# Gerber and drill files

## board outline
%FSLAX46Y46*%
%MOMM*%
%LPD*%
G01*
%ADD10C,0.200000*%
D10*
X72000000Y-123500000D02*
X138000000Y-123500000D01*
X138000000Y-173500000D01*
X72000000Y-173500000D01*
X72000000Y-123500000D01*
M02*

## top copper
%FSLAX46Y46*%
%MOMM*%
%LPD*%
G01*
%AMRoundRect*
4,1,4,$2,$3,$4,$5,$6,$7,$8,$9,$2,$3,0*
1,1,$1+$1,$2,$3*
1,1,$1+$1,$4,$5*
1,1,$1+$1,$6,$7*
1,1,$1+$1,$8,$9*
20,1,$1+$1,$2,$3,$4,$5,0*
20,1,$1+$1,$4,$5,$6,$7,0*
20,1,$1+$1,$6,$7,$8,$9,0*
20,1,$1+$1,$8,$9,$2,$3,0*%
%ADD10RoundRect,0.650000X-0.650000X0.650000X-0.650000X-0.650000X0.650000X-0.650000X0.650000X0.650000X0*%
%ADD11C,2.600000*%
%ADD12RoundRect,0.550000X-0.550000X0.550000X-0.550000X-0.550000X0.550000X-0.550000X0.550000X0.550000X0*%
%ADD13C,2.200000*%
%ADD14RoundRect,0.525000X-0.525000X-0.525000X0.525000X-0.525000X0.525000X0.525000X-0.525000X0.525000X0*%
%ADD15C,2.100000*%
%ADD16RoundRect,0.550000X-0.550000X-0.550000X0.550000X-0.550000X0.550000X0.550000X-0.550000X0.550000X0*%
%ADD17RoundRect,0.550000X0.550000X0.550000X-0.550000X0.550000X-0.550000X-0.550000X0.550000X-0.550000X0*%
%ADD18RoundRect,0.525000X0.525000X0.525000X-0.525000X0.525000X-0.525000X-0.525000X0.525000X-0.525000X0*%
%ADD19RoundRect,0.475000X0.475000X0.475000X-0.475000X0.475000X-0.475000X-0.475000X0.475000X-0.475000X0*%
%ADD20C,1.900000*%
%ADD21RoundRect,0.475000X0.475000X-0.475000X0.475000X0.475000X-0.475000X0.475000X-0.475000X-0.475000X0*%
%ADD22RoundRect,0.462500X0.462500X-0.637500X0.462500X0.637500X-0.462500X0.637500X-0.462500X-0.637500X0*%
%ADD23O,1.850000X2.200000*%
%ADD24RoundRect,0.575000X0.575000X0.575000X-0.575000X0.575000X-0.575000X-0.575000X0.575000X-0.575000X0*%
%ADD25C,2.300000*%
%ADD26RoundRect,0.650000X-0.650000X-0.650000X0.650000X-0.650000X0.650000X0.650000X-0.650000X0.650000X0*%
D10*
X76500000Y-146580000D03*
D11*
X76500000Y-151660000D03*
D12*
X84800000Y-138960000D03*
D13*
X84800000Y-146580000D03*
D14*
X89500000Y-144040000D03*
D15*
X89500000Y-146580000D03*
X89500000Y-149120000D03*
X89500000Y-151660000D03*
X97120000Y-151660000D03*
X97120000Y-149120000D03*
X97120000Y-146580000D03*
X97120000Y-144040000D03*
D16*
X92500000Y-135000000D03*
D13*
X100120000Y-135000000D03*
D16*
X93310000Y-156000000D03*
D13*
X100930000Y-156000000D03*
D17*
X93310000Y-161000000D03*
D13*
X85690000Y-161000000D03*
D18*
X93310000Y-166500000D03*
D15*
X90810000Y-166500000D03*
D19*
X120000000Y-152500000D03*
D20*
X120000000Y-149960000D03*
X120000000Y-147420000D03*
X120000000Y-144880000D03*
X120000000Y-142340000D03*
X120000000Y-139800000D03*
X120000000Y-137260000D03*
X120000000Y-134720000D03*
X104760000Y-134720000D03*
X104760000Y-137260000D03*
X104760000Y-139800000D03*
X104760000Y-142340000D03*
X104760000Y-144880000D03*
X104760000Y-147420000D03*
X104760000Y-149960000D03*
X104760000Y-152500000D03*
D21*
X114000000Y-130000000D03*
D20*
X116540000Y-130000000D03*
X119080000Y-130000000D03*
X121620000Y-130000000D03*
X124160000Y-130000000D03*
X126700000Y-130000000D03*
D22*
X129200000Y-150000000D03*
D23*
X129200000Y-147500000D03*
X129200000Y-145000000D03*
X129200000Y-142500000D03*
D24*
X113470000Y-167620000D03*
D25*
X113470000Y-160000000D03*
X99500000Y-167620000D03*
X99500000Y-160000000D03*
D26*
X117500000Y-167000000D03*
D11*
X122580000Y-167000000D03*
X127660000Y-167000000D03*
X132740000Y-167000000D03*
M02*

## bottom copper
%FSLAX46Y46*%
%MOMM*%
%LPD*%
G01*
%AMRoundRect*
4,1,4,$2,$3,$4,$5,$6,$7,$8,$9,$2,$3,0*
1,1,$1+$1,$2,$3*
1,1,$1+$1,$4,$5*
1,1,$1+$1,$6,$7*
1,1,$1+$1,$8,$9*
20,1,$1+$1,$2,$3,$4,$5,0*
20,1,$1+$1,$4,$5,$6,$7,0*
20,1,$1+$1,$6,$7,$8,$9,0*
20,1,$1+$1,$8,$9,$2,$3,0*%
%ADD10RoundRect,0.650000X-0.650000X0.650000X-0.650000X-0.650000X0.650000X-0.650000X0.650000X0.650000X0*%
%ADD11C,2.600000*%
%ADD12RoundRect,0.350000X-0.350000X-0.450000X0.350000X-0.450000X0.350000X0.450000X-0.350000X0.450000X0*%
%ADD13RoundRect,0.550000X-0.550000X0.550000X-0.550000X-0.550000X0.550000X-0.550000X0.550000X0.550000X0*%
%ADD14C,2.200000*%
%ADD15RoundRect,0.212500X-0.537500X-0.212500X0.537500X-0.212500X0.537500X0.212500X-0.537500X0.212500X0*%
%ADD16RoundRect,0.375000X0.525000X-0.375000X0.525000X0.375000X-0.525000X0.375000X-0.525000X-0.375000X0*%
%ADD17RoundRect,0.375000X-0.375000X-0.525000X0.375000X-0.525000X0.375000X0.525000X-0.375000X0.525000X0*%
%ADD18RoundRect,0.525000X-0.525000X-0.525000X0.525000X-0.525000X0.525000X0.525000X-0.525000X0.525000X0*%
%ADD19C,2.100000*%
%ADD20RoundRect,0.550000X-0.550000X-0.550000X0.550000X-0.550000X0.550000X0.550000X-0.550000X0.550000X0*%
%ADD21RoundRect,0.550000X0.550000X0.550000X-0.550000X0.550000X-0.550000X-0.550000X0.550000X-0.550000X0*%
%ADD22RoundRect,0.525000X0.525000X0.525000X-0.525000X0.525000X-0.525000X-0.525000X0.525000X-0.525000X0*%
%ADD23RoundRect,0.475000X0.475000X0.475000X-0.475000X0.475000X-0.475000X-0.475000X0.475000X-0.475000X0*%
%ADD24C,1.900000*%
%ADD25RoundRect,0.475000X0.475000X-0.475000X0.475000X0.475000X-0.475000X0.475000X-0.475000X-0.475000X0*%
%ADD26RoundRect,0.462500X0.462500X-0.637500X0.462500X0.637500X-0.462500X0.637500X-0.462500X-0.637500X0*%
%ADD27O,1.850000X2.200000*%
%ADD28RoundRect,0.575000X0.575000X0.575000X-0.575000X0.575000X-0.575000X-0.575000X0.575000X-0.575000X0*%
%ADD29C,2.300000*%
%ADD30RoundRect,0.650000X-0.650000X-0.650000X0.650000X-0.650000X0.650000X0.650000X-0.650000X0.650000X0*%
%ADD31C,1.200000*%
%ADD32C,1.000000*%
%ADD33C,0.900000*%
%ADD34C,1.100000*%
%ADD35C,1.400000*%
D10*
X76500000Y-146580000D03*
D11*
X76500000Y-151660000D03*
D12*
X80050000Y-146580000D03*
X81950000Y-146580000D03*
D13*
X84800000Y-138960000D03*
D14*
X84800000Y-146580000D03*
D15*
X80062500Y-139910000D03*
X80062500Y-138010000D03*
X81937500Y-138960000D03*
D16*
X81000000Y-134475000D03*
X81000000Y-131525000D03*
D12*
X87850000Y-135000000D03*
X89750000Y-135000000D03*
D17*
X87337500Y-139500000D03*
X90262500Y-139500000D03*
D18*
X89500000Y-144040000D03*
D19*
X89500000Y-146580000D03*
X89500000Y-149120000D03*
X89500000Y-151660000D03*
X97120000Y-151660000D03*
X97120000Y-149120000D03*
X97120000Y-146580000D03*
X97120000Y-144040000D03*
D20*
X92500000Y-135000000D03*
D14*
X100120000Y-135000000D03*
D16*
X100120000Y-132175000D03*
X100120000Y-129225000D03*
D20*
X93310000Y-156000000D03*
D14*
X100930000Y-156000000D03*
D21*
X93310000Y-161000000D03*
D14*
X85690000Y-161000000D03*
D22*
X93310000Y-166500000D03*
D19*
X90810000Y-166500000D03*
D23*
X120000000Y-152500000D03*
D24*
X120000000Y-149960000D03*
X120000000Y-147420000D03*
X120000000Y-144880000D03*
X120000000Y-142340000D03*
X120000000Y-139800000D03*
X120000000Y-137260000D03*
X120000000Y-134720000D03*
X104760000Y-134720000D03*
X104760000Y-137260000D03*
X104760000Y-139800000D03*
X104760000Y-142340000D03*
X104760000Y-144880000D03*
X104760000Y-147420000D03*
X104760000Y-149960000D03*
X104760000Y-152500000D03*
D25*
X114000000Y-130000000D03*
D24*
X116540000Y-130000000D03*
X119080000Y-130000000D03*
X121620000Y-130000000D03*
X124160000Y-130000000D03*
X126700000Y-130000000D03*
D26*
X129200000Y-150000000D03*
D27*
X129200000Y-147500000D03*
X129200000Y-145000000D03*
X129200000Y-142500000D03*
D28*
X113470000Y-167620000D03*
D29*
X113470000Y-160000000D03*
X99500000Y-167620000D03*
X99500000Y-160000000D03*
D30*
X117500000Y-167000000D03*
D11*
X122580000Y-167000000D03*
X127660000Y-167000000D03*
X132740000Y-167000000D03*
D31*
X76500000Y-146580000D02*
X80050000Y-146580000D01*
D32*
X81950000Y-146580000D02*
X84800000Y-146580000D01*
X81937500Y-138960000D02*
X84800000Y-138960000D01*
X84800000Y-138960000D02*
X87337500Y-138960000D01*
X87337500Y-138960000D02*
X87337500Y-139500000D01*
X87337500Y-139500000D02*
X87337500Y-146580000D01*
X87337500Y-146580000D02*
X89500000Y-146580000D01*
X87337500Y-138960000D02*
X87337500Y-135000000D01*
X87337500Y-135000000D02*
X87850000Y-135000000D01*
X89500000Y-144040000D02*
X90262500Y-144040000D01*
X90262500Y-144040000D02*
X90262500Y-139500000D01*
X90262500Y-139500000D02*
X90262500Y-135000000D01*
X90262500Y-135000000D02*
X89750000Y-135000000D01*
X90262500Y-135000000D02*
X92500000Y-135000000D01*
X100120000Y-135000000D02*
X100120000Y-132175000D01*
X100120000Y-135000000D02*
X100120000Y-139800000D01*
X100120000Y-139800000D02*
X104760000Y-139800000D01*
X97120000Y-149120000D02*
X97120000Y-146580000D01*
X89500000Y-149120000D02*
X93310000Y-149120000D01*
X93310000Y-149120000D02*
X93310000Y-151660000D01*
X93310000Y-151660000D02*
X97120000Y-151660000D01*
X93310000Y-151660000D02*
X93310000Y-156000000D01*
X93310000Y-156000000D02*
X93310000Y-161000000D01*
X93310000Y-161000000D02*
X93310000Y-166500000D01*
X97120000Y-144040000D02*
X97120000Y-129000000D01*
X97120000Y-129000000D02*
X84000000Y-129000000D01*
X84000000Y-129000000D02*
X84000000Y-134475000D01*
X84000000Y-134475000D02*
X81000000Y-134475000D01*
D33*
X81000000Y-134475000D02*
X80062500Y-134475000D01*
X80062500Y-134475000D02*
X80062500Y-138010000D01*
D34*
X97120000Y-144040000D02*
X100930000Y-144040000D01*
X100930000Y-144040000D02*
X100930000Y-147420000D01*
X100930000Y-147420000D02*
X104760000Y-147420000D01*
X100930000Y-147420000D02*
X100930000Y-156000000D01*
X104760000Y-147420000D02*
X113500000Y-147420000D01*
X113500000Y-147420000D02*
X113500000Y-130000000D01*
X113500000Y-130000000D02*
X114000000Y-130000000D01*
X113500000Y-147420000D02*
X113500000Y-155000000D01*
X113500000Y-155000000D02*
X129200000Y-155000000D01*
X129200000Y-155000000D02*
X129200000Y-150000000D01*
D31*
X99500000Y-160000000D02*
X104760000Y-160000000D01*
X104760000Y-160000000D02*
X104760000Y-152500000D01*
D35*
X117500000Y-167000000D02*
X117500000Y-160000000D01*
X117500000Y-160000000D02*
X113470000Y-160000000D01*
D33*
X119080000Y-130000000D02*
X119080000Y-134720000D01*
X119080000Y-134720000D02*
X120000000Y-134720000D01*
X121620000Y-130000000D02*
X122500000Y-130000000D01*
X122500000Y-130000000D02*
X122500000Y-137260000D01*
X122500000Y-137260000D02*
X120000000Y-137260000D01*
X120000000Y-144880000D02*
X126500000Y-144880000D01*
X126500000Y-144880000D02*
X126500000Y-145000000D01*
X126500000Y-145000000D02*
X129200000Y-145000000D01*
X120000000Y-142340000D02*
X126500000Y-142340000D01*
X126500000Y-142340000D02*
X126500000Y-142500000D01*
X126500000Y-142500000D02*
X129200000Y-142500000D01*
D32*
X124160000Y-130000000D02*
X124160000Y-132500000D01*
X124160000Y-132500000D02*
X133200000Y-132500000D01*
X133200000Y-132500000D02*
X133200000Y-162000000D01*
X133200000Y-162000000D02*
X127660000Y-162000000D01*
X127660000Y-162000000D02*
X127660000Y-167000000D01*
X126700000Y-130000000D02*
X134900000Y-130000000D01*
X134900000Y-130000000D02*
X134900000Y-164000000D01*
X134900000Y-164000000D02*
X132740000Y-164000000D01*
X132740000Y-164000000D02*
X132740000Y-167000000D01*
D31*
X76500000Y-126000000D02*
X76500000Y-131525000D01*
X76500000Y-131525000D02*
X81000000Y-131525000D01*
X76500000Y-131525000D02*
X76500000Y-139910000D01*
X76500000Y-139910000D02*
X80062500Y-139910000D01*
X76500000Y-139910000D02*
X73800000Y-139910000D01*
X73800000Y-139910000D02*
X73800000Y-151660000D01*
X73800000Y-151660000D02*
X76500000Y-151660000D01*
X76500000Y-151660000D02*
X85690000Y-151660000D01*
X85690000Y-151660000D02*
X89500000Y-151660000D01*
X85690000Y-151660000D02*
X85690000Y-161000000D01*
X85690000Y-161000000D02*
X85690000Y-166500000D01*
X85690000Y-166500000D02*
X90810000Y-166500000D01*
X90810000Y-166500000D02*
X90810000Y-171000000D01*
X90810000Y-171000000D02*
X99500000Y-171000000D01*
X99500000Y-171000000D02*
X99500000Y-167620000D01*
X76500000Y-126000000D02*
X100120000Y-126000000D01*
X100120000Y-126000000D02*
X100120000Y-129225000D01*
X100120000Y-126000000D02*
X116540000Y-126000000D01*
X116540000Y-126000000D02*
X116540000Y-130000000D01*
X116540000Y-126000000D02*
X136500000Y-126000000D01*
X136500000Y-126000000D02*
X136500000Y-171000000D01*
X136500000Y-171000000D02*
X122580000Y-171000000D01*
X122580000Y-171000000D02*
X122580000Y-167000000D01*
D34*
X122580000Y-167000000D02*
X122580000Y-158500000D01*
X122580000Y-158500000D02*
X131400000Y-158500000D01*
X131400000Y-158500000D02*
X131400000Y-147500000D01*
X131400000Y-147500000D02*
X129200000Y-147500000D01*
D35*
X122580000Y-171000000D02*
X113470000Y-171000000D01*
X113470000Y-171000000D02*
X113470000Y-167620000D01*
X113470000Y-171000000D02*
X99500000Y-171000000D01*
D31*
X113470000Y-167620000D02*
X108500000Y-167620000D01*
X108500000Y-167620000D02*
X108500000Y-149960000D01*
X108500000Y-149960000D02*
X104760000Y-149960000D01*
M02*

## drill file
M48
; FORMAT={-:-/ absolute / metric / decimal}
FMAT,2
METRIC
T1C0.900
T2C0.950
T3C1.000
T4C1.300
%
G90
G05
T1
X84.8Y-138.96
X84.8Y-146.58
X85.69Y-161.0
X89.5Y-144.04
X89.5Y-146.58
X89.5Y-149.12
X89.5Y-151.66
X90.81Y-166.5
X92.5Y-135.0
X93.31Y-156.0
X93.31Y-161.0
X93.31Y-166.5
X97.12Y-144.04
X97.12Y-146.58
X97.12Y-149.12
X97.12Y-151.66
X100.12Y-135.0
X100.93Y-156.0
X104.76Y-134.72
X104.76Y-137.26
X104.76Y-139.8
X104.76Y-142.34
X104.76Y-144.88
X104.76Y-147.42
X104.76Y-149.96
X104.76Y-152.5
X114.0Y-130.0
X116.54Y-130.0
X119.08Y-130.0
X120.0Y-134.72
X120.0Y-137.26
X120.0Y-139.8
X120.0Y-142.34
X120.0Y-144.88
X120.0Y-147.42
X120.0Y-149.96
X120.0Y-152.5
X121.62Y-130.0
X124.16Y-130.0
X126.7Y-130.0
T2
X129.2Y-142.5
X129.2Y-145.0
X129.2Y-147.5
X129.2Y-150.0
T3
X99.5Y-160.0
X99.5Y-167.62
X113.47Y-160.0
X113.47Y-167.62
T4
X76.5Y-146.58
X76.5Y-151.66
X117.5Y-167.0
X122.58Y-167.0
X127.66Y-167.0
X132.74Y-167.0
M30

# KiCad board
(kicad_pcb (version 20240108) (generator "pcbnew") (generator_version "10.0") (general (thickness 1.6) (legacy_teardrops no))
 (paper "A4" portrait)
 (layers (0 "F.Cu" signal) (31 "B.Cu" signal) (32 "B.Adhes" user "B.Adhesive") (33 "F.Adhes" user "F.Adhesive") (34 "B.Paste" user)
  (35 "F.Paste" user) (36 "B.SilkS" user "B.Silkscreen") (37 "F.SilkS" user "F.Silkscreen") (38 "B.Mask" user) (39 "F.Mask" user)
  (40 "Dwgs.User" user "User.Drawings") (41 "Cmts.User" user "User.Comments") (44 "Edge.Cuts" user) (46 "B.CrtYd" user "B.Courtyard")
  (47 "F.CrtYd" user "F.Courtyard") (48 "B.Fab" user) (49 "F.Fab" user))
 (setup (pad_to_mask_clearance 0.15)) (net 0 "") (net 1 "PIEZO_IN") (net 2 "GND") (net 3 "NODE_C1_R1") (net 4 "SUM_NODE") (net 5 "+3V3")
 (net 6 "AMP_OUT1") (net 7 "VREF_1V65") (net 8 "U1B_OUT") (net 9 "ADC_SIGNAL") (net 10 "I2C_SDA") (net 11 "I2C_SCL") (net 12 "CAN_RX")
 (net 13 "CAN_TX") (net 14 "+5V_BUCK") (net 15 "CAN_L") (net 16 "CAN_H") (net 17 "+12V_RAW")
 (gr_rect (start 72.000 123.500) (end 138.000 173.500) (stroke (width 0.2) (type default)) (fill none) (layer "Edge.Cuts"))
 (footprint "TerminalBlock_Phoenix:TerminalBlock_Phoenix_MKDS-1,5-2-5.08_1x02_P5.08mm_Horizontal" (layer "F.Cu") (at 76.5000 146.5800 270)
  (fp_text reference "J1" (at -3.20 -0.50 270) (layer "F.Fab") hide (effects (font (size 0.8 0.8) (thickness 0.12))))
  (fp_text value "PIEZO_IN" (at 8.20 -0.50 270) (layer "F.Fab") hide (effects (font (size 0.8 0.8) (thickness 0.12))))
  (pad "1" thru_hole roundrect (at 0.0000 0.0000 270) (size 2.60 2.60) (drill 1.30) (layers "*.Cu" "*.Mask") (roundrect_rratio 0.25)
   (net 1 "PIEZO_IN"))
  (pad "2" thru_hole circle (at 5.0800 0.0000 270) (size 2.60 2.60) (drill 1.30) (layers "*.Cu" "*.Mask") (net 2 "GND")))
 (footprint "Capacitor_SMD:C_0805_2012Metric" (layer "B.Cu") (at 81.0000 146.5800 0)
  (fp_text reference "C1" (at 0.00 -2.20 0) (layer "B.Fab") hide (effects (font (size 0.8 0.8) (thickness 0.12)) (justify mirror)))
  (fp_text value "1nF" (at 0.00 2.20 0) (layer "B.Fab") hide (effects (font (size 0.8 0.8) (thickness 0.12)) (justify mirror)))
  (pad "1" smd roundrect (at -0.9500 0.0000 0) (size 1.40 1.60) (layers "B.Cu" "B.Mask" "B.Paste") (roundrect_rratio 0.25)
   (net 1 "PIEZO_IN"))
  (pad "2" smd roundrect (at 0.9500 0.0000 0) (size 1.40 1.60) (layers "B.Cu" "B.Mask" "B.Paste") (roundrect_rratio 0.25)
   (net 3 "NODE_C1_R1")))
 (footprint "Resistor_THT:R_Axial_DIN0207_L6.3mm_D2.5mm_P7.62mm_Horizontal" (layer "F.Cu") (at 84.8000 138.9600 270)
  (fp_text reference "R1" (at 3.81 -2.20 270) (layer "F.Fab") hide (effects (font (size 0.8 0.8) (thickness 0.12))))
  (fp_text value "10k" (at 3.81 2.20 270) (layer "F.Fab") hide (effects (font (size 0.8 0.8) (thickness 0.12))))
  (pad "1" thru_hole roundrect (at 0.0000 0.0000 270) (size 2.20 2.20) (drill 0.90) (layers "*.Cu" "*.Mask") (roundrect_rratio 0.25)
   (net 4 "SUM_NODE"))
  (pad "2" thru_hole circle (at 7.6200 0.0000 270) (size 2.20 2.20) (drill 0.90) (layers "*.Cu" "*.Mask") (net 3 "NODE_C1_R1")))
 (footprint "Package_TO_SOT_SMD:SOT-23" (layer "B.Cu") (at 81.0000 138.9600 0)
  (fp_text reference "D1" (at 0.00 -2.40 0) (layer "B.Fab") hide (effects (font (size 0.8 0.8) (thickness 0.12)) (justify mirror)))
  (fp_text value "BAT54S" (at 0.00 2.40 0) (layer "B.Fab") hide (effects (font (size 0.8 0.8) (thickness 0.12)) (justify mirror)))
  (pad "1" smd roundrect (at -0.9375 0.9500 0) (size 1.50 0.85) (layers "B.Cu" "B.Mask" "B.Paste") (roundrect_rratio 0.25) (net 2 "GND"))
  (pad "2" smd roundrect (at -0.9375 -0.9500 0) (size 1.50 0.85) (layers "B.Cu" "B.Mask" "B.Paste") (roundrect_rratio 0.25) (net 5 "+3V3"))
  (pad "3" smd roundrect (at 0.9375 0.0000 0) (size 1.50 0.85) (layers "B.Cu" "B.Mask" "B.Paste") (roundrect_rratio 0.25) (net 4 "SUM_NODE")))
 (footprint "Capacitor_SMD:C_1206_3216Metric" (layer "B.Cu") (at 81.0000 133.0000 90)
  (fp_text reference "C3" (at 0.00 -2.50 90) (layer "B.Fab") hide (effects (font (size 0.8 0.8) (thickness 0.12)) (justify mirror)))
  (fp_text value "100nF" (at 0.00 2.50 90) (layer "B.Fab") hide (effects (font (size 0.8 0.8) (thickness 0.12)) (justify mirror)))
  (pad "1" smd roundrect (at -1.4750 0.0000 90) (size 1.50 1.80) (layers "B.Cu" "B.Mask" "B.Paste") (roundrect_rratio 0.25) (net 5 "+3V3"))
  (pad "2" smd roundrect (at 1.4750 0.0000 90) (size 1.50 1.80) (layers "B.Cu" "B.Mask" "B.Paste") (roundrect_rratio 0.25) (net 2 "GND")))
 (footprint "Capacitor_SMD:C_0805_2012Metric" (layer "B.Cu") (at 88.8000 135.0000 0)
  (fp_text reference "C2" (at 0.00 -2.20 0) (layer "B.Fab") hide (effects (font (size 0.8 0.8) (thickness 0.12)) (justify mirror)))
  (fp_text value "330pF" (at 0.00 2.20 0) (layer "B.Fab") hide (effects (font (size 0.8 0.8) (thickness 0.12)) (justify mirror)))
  (pad "1" smd roundrect (at -0.9500 0.0000 0) (size 1.40 1.60) (layers "B.Cu" "B.Mask" "B.Paste") (roundrect_rratio 0.25)
   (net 4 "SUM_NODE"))
  (pad "2" smd roundrect (at 0.9500 0.0000 0) (size 1.40 1.60) (layers "B.Cu" "B.Mask" "B.Paste") (roundrect_rratio 0.25) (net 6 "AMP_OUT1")))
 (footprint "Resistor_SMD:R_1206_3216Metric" (layer "B.Cu") (at 88.8000 139.5000 0)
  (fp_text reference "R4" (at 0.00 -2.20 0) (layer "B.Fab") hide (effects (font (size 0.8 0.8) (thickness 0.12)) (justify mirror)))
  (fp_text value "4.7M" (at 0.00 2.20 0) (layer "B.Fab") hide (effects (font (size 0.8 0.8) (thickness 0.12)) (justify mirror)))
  (pad "1" smd roundrect (at -1.4625 0.0000 0) (size 1.50 1.80) (layers "B.Cu" "B.Mask" "B.Paste") (roundrect_rratio 0.25)
   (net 4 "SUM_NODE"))
  (pad "2" smd roundrect (at 1.4625 0.0000 0) (size 1.50 1.80) (layers "B.Cu" "B.Mask" "B.Paste") (roundrect_rratio 0.25) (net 6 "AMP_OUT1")))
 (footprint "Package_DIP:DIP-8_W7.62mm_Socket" (layer "F.Cu") (at 89.5000 144.0400 0)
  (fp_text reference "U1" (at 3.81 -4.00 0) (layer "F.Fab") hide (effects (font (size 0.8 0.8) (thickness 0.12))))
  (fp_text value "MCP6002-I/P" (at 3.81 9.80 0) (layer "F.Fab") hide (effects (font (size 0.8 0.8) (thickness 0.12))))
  (pad "1" thru_hole roundrect (at 0.0000 0.0000 0) (size 2.10 2.10) (drill 0.90) (layers "*.Cu" "*.Mask") (roundrect_rratio 0.25)
   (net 6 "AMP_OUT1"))
  (pad "2" thru_hole circle (at 0.0000 2.5400 0) (size 2.10 2.10) (drill 0.90) (layers "*.Cu" "*.Mask") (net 4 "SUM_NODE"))
  (pad "3" thru_hole circle (at 0.0000 5.0800 0) (size 2.10 2.10) (drill 0.90) (layers "*.Cu" "*.Mask") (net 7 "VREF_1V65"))
  (pad "4" thru_hole circle (at 0.0000 7.6200 0) (size 2.10 2.10) (drill 0.90) (layers "*.Cu" "*.Mask") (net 2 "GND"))
  (pad "5" thru_hole circle (at 7.6200 7.6200 0) (size 2.10 2.10) (drill 0.90) (layers "*.Cu" "*.Mask") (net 7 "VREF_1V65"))
  (pad "6" thru_hole circle (at 7.6200 5.0800 0) (size 2.10 2.10) (drill 0.90) (layers "*.Cu" "*.Mask") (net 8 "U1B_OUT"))
  (pad "7" thru_hole circle (at 7.6200 2.5400 0) (size 2.10 2.10) (drill 0.90) (layers "*.Cu" "*.Mask") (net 8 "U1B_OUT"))
  (pad "8" thru_hole circle (at 7.6200 0.0000 0) (size 2.10 2.10) (drill 0.90) (layers "*.Cu" "*.Mask") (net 5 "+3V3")))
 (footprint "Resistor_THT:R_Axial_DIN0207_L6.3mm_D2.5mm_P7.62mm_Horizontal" (layer "F.Cu") (at 92.5000 135.0000 0)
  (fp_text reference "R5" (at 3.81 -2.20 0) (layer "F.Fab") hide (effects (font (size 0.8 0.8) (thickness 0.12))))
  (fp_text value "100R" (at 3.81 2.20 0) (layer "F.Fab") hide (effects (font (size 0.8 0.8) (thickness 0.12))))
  (pad "1" thru_hole roundrect (at 0.0000 0.0000 0) (size 2.20 2.20) (drill 0.90) (layers "*.Cu" "*.Mask") (roundrect_rratio 0.25)
   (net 6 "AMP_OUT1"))
  (pad "2" thru_hole circle (at 7.6200 0.0000 0) (size 2.20 2.20) (drill 0.90) (layers "*.Cu" "*.Mask") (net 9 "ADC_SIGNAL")))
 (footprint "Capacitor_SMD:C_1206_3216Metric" (layer "B.Cu") (at 100.1200 130.7000 90)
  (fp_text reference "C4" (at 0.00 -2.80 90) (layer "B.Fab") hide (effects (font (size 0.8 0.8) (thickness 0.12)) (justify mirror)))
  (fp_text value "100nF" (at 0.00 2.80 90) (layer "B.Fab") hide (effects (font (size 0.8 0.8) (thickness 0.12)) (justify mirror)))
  (pad "1" smd roundrect (at -1.4750 0.0000 90) (size 1.50 1.80) (layers "B.Cu" "B.Mask" "B.Paste") (roundrect_rratio 0.25)
   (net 9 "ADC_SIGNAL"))
  (pad "2" smd roundrect (at 1.4750 0.0000 90) (size 1.50 1.80) (layers "B.Cu" "B.Mask" "B.Paste") (roundrect_rratio 0.25) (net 2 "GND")))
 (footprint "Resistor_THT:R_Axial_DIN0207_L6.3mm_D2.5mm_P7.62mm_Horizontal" (layer "F.Cu") (at 93.3100 156.0000 0)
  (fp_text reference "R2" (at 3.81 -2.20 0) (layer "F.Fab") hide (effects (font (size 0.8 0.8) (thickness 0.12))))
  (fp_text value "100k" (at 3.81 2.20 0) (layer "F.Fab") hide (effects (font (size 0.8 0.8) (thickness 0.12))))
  (pad "1" thru_hole roundrect (at 0.0000 0.0000 0) (size 2.20 2.20) (drill 0.90) (layers "*.Cu" "*.Mask") (roundrect_rratio 0.25)
   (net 7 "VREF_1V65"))
  (pad "2" thru_hole circle (at 7.6200 0.0000 0) (size 2.20 2.20) (drill 0.90) (layers "*.Cu" "*.Mask") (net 5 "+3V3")))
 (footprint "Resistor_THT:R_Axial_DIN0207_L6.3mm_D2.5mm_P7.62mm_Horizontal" (layer "F.Cu") (at 93.3100 161.0000 180)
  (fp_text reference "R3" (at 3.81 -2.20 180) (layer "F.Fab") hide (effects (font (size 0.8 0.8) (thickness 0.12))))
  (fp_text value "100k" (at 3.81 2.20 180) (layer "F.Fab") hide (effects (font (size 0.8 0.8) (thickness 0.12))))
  (pad "1" thru_hole roundrect (at 0.0000 0.0000 180) (size 2.20 2.20) (drill 0.90) (layers "*.Cu" "*.Mask") (roundrect_rratio 0.25)
   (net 7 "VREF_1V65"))
  (pad "2" thru_hole circle (at 7.6200 0.0000 180) (size 2.20 2.20) (drill 0.90) (layers "*.Cu" "*.Mask") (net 2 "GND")))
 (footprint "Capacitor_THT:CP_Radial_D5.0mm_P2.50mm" (layer "F.Cu") (at 93.3100 166.5000 180)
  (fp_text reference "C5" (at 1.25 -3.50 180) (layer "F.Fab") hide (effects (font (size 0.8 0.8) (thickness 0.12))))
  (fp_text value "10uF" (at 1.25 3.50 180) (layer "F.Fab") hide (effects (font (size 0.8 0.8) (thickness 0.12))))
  (pad "1" thru_hole roundrect (at 0.0000 0.0000 180) (size 2.10 2.10) (drill 0.90) (layers "*.Cu" "*.Mask") (roundrect_rratio 0.25)
   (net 7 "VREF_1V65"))
  (pad "2" thru_hole circle (at 2.5000 0.0000 180) (size 2.10 2.10) (drill 0.90) (layers "*.Cu" "*.Mask") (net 2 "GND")))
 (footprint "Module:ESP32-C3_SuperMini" (layer "F.Cu") (at 120.0000 152.5000 180)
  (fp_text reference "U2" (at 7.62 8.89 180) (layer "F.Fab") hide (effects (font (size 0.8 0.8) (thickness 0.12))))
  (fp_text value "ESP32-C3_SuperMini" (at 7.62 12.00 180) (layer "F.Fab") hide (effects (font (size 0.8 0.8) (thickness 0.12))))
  (pad "1" thru_hole roundrect (at 0.0000 0.0000 180) (size 1.90 1.90) (drill 0.90) (layers "*.Cu" "*.Mask") (roundrect_rratio 0.25))
  (pad "2" thru_hole circle (at 0.0000 2.5400 180) (size 1.90 1.90) (drill 0.90) (layers "*.Cu" "*.Mask"))
  (pad "3" thru_hole circle (at 0.0000 5.0800 180) (size 1.90 1.90) (drill 0.90) (layers "*.Cu" "*.Mask"))
  (pad "4" thru_hole circle (at 0.0000 7.6200 180) (size 1.90 1.90) (drill 0.90) (layers "*.Cu" "*.Mask") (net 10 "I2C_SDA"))
  (pad "5" thru_hole circle (at 0.0000 10.1600 180) (size 1.90 1.90) (drill 0.90) (layers "*.Cu" "*.Mask") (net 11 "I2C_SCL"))
  (pad "6" thru_hole circle (at 0.0000 12.7000 180) (size 1.90 1.90) (drill 0.90) (layers "*.Cu" "*.Mask"))
  (pad "7" thru_hole circle (at 0.0000 15.2400 180) (size 1.90 1.90) (drill 0.90) (layers "*.Cu" "*.Mask") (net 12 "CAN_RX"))
  (pad "8" thru_hole circle (at 0.0000 17.7800 180) (size 1.90 1.90) (drill 0.90) (layers "*.Cu" "*.Mask") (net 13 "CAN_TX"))
  (pad "9" thru_hole circle (at 15.2400 17.7800 180) (size 1.90 1.90) (drill 0.90) (layers "*.Cu" "*.Mask"))
  (pad "10" thru_hole circle (at 15.2400 15.2400 180) (size 1.90 1.90) (drill 0.90) (layers "*.Cu" "*.Mask"))
  (pad "11" thru_hole circle (at 15.2400 12.7000 180) (size 1.90 1.90) (drill 0.90) (layers "*.Cu" "*.Mask") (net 9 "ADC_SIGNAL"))
  (pad "12" thru_hole circle (at 15.2400 10.1600 180) (size 1.90 1.90) (drill 0.90) (layers "*.Cu" "*.Mask"))
  (pad "13" thru_hole circle (at 15.2400 7.6200 180) (size 1.90 1.90) (drill 0.90) (layers "*.Cu" "*.Mask"))
  (pad "14" thru_hole circle (at 15.2400 5.0800 180) (size 1.90 1.90) (drill 0.90) (layers "*.Cu" "*.Mask") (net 5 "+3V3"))
  (pad "15" thru_hole circle (at 15.2400 2.5400 180) (size 1.90 1.90) (drill 0.90) (layers "*.Cu" "*.Mask") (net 2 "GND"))
  (pad "16" thru_hole circle (at 15.2400 0.0000 180) (size 1.90 1.90) (drill 0.90) (layers "*.Cu" "*.Mask") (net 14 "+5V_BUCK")))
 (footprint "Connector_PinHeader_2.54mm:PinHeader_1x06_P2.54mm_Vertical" (layer "F.Cu") (at 114.0000 130.0000 90)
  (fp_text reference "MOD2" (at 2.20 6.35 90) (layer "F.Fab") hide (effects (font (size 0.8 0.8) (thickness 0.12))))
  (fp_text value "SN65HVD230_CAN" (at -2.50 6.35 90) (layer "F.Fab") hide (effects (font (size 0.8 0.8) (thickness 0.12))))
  (pad "1" thru_hole roundrect (at 0.0000 0.0000 90) (size 1.90 1.90) (drill 0.90) (layers "*.Cu" "*.Mask") (roundrect_rratio 0.25)
   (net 5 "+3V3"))
  (pad "2" thru_hole circle (at 0.0000 2.5400 90) (size 1.90 1.90) (drill 0.90) (layers "*.Cu" "*.Mask") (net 2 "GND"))
  (pad "3" thru_hole circle (at 0.0000 5.0800 90) (size 1.90 1.90) (drill 0.90) (layers "*.Cu" "*.Mask") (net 13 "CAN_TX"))
  (pad "4" thru_hole circle (at 0.0000 7.6200 90) (size 1.90 1.90) (drill 0.90) (layers "*.Cu" "*.Mask") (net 12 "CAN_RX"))
  (pad "5" thru_hole circle (at 0.0000 10.1600 90) (size 1.90 1.90) (drill 0.90) (layers "*.Cu" "*.Mask") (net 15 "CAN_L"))
  (pad "6" thru_hole circle (at 0.0000 12.7000 90) (size 1.90 1.90) (drill 0.90) (layers "*.Cu" "*.Mask") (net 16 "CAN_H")))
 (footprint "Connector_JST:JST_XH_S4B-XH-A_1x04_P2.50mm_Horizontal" (layer "F.Cu") (at 129.2000 150.0000 90)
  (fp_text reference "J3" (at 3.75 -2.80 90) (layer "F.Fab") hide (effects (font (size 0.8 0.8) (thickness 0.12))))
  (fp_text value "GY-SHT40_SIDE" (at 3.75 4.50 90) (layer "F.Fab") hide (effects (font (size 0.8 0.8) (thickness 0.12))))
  (pad "1" thru_hole roundrect (at 0.0000 0.0000 90) (size 2.20 1.85) (drill 0.95) (layers "*.Cu" "*.Mask") (roundrect_rratio 0.25)
   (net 5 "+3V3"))
  (pad "2" thru_hole oval (at 2.5000 0.0000 90) (size 2.20 1.85) (drill 0.95) (layers "*.Cu" "*.Mask") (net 2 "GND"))
  (pad "3" thru_hole oval (at 5.0000 0.0000 90) (size 2.20 1.85) (drill 0.95) (layers "*.Cu" "*.Mask") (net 10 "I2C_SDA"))
  (pad "4" thru_hole oval (at 7.5000 0.0000 90) (size 2.20 1.85) (drill 0.95) (layers "*.Cu" "*.Mask") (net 11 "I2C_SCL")))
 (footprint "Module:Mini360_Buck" (layer "F.Cu") (at 113.4700 167.6200 180)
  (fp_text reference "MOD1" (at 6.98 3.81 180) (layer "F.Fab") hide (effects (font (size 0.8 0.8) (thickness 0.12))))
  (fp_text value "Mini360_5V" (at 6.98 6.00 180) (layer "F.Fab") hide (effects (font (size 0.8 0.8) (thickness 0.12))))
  (pad "1" thru_hole roundrect (at 0.0000 0.0000 180) (size 2.30 2.30) (drill 1.00) (layers "*.Cu" "*.Mask") (roundrect_rratio 0.25)
   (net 2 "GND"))
  (pad "2" thru_hole circle (at 0.0000 7.6200 180) (size 2.30 2.30) (drill 1.00) (layers "*.Cu" "*.Mask") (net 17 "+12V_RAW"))
  (pad "3" thru_hole circle (at 13.9700 0.0000 180) (size 2.30 2.30) (drill 1.00) (layers "*.Cu" "*.Mask") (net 2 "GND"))
  (pad "4" thru_hole circle (at 13.9700 7.6200 180) (size 2.30 2.30) (drill 1.00) (layers "*.Cu" "*.Mask") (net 14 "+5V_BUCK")))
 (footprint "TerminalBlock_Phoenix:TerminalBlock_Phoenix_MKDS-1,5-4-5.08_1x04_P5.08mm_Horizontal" (layer "F.Cu") (at 117.5000 167.0000 0)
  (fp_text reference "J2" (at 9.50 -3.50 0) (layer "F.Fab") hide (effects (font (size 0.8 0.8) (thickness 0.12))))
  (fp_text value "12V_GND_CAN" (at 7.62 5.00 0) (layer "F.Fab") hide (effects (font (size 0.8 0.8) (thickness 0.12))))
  (pad "1" thru_hole roundrect (at 0.0000 0.0000 0) (size 2.60 2.60) (drill 1.30) (layers "*.Cu" "*.Mask") (roundrect_rratio 0.25)
   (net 17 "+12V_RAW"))
  (pad "2" thru_hole circle (at 5.0800 0.0000 0) (size 2.60 2.60) (drill 1.30) (layers "*.Cu" "*.Mask") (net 2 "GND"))
  (pad "3" thru_hole circle (at 10.1600 0.0000 0) (size 2.60 2.60) (drill 1.30) (layers "*.Cu" "*.Mask") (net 15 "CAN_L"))
  (pad "4" thru_hole circle (at 15.2400 0.0000 0) (size 2.60 2.60) (drill 1.30) (layers "*.Cu" "*.Mask") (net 16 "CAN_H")))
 (segment (start 76.5000 146.5800) (end 80.0500 146.5800) (width 1.20) (layer "B.Cu") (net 1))
 (segment (start 81.9500 146.5800) (end 84.8000 146.5800) (width 1.00) (layer "B.Cu") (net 3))
 (segment (start 81.9375 138.9600) (end 84.8000 138.9600) (width 1.00) (layer "B.Cu") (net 4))
 (segment (start 84.8000 138.9600) (end 87.3375 138.9600) (width 1.00) (layer "B.Cu") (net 4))
 (segment (start 87.3375 138.9600) (end 87.3375 139.5000) (width 1.00) (layer "B.Cu") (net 4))
 (segment (start 87.3375 139.5000) (end 87.3375 146.5800) (width 1.00) (layer "B.Cu") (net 4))
 (segment (start 87.3375 146.5800) (end 89.5000 146.5800) (width 1.00) (layer "B.Cu") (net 4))
 (segment (start 87.3375 138.9600) (end 87.3375 135.0000) (width 1.00) (layer "B.Cu") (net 4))
 (segment (start 87.3375 135.0000) (end 87.8500 135.0000) (width 1.00) (layer "B.Cu") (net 4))
 (segment (start 89.5000 144.0400) (end 90.2625 144.0400) (width 1.00) (layer "B.Cu") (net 6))
 (segment (start 90.2625 144.0400) (end 90.2625 139.5000) (width 1.00) (layer "B.Cu") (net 6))
 (segment (start 90.2625 139.5000) (end 90.2625 135.0000) (width 1.00) (layer "B.Cu") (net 6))
 (segment (start 90.2625 135.0000) (end 89.7500 135.0000) (width 1.00) (layer "B.Cu") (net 6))
 (segment (start 90.2625 135.0000) (end 92.5000 135.0000) (width 1.00) (layer "B.Cu") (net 6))
 (segment (start 100.1200 135.0000) (end 100.1200 132.1750) (width 1.00) (layer "B.Cu") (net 9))
 (segment (start 100.1200 135.0000) (end 100.1200 139.8000) (width 1.00) (layer "B.Cu") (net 9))
 (segment (start 100.1200 139.8000) (end 104.7600 139.8000) (width 1.00) (layer "B.Cu") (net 9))
 (segment (start 97.1200 149.1200) (end 97.1200 146.5800) (width 1.00) (layer "B.Cu") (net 8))
 (segment (start 89.5000 149.1200) (end 93.3100 149.1200) (width 1.00) (layer "B.Cu") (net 7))
 (segment (start 93.3100 149.1200) (end 93.3100 151.6600) (width 1.00) (layer "B.Cu") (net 7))
 (segment (start 93.3100 151.6600) (end 97.1200 151.6600) (width 1.00) (layer "B.Cu") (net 7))
 (segment (start 93.3100 151.6600) (end 93.3100 156.0000) (width 1.00) (layer "B.Cu") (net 7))
 (segment (start 93.3100 156.0000) (end 93.3100 161.0000) (width 1.00) (layer "B.Cu") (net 7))
 (segment (start 93.3100 161.0000) (end 93.3100 166.5000) (width 1.00) (layer "B.Cu") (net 7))
 (segment (start 97.1200 144.0400) (end 97.1200 129.0000) (width 1.00) (layer "B.Cu") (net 5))
 (segment (start 97.1200 129.0000) (end 84.0000 129.0000) (width 1.00) (layer "B.Cu") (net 5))
 (segment (start 84.0000 129.0000) (end 84.0000 134.4750) (width 1.00) (layer "B.Cu") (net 5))
 (segment (start 84.0000 134.4750) (end 81.0000 134.4750) (width 1.00) (layer "B.Cu") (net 5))
 (segment (start 81.0000 134.4750) (end 80.0625 134.4750) (width 0.90) (layer "B.Cu") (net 5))
 (segment (start 80.0625 134.4750) (end 80.0625 138.0100) (width 0.90) (layer "B.Cu") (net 5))
 (segment (start 97.1200 144.0400) (end 100.9300 144.0400) (width 1.10) (layer "B.Cu") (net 5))
 (segment (start 100.9300 144.0400) (end 100.9300 147.4200) (width 1.10) (layer "B.Cu") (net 5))
 (segment (start 100.9300 147.4200) (end 104.7600 147.4200) (width 1.10) (layer "B.Cu") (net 5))
 (segment (start 100.9300 147.4200) (end 100.9300 156.0000) (width 1.10) (layer "B.Cu") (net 5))
 (segment (start 104.7600 147.4200) (end 113.5000 147.4200) (width 1.10) (layer "B.Cu") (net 5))
 (segment (start 113.5000 147.4200) (end 113.5000 130.0000) (width 1.10) (layer "B.Cu") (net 5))
 (segment (start 113.5000 130.0000) (end 114.0000 130.0000) (width 1.10) (layer "B.Cu") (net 5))
 (segment (start 113.5000 147.4200) (end 113.5000 155.0000) (width 1.10) (layer "B.Cu") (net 5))
 (segment (start 113.5000 155.0000) (end 129.2000 155.0000) (width 1.10) (layer "B.Cu") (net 5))
 (segment (start 129.2000 155.0000) (end 129.2000 150.0000) (width 1.10) (layer "B.Cu") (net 5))
 (segment (start 99.5000 160.0000) (end 104.7600 160.0000) (width 1.20) (layer "B.Cu") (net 14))
 (segment (start 104.7600 160.0000) (end 104.7600 152.5000) (width 1.20) (layer "B.Cu") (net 14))
 (segment (start 117.5000 167.0000) (end 117.5000 160.0000) (width 1.40) (layer "B.Cu") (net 17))
 (segment (start 117.5000 160.0000) (end 113.4700 160.0000) (width 1.40) (layer "B.Cu") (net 17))
 (segment (start 119.0800 130.0000) (end 119.0800 134.7200) (width 0.90) (layer "B.Cu") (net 13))
 (segment (start 119.0800 134.7200) (end 120.0000 134.7200) (width 0.90) (layer "B.Cu") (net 13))
 (segment (start 121.6200 130.0000) (end 122.5000 130.0000) (width 0.90) (layer "B.Cu") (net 12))
 (segment (start 122.5000 130.0000) (end 122.5000 137.2600) (width 0.90) (layer "B.Cu") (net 12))
 (segment (start 122.5000 137.2600) (end 120.0000 137.2600) (width 0.90) (layer "B.Cu") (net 12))
 (segment (start 120.0000 144.8800) (end 126.5000 144.8800) (width 0.90) (layer "B.Cu") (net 10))
 (segment (start 126.5000 144.8800) (end 126.5000 145.0000) (width 0.90) (layer "B.Cu") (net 10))
 (segment (start 126.5000 145.0000) (end 129.2000 145.0000) (width 0.90) (layer "B.Cu") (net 10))
 (segment (start 120.0000 142.3400) (end 126.5000 142.3400) (width 0.90) (layer "B.Cu") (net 11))
 (segment (start 126.5000 142.3400) (end 126.5000 142.5000) (width 0.90) (layer "B.Cu") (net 11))
 (segment (start 126.5000 142.5000) (end 129.2000 142.5000) (width 0.90) (layer "B.Cu") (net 11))
 (segment (start 124.1600 130.0000) (end 124.1600 132.5000) (width 1.00) (layer "B.Cu") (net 15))
 (segment (start 124.1600 132.5000) (end 133.2000 132.5000) (width 1.00) (layer "B.Cu") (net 15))
 (segment (start 133.2000 132.5000) (end 133.2000 162.0000) (width 1.00) (layer "B.Cu") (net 15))
 (segment (start 133.2000 162.0000) (end 127.6600 162.0000) (width 1.00) (layer "B.Cu") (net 15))
 (segment (start 127.6600 162.0000) (end 127.6600 167.0000) (width 1.00) (layer "B.Cu") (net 15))
 (segment (start 126.7000 130.0000) (end 134.9000 130.0000) (width 1.00) (layer "B.Cu") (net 16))
 (segment (start 134.9000 130.0000) (end 134.9000 164.0000) (width 1.00) (layer "B.Cu") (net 16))
 (segment (start 134.9000 164.0000) (end 132.7400 164.0000) (width 1.00) (layer "B.Cu") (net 16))
 (segment (start 132.7400 164.0000) (end 132.7400 167.0000) (width 1.00) (layer "B.Cu") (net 16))
 (segment (start 76.5000 126.0000) (end 76.5000 131.5250) (width 1.20) (layer "B.Cu") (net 2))
 (segment (start 76.5000 131.5250) (end 81.0000 131.5250) (width 1.20) (layer "B.Cu") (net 2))
 (segment (start 76.5000 131.5250) (end 76.5000 139.9100) (width 1.20) (layer "B.Cu") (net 2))
 (segment (start 76.5000 139.9100) (end 80.0625 139.9100) (width 1.20) (layer "B.Cu") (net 2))
 (segment (start 76.5000 139.9100) (end 73.8000 139.9100) (width 1.20) (layer "B.Cu") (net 2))
 (segment (start 73.8000 139.9100) (end 73.8000 151.6600) (width 1.20) (layer "B.Cu") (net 2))
 (segment (start 73.8000 151.6600) (end 76.5000 151.6600) (width 1.20) (layer "B.Cu") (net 2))
 (segment (start 76.5000 151.6600) (end 85.6900 151.6600) (width 1.20) (layer "B.Cu") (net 2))
 (segment (start 85.6900 151.6600) (end 89.5000 151.6600) (width 1.20) (layer "B.Cu") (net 2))
 (segment (start 85.6900 151.6600) (end 85.6900 161.0000) (width 1.20) (layer "B.Cu") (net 2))
 (segment (start 85.6900 161.0000) (end 85.6900 166.5000) (width 1.20) (layer "B.Cu") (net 2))
 (segment (start 85.6900 166.5000) (end 90.8100 166.5000) (width 1.20) (layer "B.Cu") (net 2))
 (segment (start 90.8100 166.5000) (end 90.8100 171.0000) (width 1.20) (layer "B.Cu") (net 2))
 (segment (start 90.8100 171.0000) (end 99.5000 171.0000) (width 1.20) (layer "B.Cu") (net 2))
 (segment (start 99.5000 171.0000) (end 99.5000 167.6200) (width 1.20) (layer "B.Cu") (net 2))
 (segment (start 76.5000 126.0000) (end 100.1200 126.0000) (width 1.20) (layer "B.Cu") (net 2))
 (segment (start 100.1200 126.0000) (end 100.1200 129.2250) (width 1.20) (layer "B.Cu") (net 2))
 (segment (start 100.1200 126.0000) (end 116.5400 126.0000) (width 1.20) (layer "B.Cu") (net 2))
 (segment (start 116.5400 126.0000) (end 116.5400 130.0000) (width 1.20) (layer "B.Cu") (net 2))
 (segment (start 116.5400 126.0000) (end 136.5000 126.0000) (width 1.20) (layer "B.Cu") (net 2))
 (segment (start 136.5000 126.0000) (end 136.5000 171.0000) (width 1.20) (layer "B.Cu") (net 2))
 (segment (start 136.5000 171.0000) (end 122.5800 171.0000) (width 1.20) (layer "B.Cu") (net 2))
 (segment (start 122.5800 171.0000) (end 122.5800 167.0000) (width 1.20) (layer "B.Cu") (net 2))
 (segment (start 122.5800 167.0000) (end 122.5800 158.5000) (width 1.10) (layer "B.Cu") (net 2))
 (segment (start 122.5800 158.5000) (end 131.4000 158.5000) (width 1.10) (layer "B.Cu") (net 2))
 (segment (start 131.4000 158.5000) (end 131.4000 147.5000) (width 1.10) (layer "B.Cu") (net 2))
 (segment (start 131.4000 147.5000) (end 129.2000 147.5000) (width 1.10) (layer "B.Cu") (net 2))
 (segment (start 122.5800 171.0000) (end 113.4700 171.0000) (width 1.40) (layer "B.Cu") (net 2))
 (segment (start 113.4700 171.0000) (end 113.4700 167.6200) (width 1.40) (layer "B.Cu") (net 2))
 (segment (start 113.4700 171.0000) (end 99.5000 171.0000) (width 1.40) (layer "B.Cu") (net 2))
 (segment (start 113.4700 167.6200) (end 108.5000 167.6200) (width 1.20) (layer "B.Cu") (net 2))
 (segment (start 108.5000 167.6200) (end 108.5000 149.9600) (width 1.20) (layer "B.Cu") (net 2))
 (segment (start 108.5000 149.9600) (end 104.7600 149.9600) (width 1.20) (layer "B.Cu") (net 2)))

